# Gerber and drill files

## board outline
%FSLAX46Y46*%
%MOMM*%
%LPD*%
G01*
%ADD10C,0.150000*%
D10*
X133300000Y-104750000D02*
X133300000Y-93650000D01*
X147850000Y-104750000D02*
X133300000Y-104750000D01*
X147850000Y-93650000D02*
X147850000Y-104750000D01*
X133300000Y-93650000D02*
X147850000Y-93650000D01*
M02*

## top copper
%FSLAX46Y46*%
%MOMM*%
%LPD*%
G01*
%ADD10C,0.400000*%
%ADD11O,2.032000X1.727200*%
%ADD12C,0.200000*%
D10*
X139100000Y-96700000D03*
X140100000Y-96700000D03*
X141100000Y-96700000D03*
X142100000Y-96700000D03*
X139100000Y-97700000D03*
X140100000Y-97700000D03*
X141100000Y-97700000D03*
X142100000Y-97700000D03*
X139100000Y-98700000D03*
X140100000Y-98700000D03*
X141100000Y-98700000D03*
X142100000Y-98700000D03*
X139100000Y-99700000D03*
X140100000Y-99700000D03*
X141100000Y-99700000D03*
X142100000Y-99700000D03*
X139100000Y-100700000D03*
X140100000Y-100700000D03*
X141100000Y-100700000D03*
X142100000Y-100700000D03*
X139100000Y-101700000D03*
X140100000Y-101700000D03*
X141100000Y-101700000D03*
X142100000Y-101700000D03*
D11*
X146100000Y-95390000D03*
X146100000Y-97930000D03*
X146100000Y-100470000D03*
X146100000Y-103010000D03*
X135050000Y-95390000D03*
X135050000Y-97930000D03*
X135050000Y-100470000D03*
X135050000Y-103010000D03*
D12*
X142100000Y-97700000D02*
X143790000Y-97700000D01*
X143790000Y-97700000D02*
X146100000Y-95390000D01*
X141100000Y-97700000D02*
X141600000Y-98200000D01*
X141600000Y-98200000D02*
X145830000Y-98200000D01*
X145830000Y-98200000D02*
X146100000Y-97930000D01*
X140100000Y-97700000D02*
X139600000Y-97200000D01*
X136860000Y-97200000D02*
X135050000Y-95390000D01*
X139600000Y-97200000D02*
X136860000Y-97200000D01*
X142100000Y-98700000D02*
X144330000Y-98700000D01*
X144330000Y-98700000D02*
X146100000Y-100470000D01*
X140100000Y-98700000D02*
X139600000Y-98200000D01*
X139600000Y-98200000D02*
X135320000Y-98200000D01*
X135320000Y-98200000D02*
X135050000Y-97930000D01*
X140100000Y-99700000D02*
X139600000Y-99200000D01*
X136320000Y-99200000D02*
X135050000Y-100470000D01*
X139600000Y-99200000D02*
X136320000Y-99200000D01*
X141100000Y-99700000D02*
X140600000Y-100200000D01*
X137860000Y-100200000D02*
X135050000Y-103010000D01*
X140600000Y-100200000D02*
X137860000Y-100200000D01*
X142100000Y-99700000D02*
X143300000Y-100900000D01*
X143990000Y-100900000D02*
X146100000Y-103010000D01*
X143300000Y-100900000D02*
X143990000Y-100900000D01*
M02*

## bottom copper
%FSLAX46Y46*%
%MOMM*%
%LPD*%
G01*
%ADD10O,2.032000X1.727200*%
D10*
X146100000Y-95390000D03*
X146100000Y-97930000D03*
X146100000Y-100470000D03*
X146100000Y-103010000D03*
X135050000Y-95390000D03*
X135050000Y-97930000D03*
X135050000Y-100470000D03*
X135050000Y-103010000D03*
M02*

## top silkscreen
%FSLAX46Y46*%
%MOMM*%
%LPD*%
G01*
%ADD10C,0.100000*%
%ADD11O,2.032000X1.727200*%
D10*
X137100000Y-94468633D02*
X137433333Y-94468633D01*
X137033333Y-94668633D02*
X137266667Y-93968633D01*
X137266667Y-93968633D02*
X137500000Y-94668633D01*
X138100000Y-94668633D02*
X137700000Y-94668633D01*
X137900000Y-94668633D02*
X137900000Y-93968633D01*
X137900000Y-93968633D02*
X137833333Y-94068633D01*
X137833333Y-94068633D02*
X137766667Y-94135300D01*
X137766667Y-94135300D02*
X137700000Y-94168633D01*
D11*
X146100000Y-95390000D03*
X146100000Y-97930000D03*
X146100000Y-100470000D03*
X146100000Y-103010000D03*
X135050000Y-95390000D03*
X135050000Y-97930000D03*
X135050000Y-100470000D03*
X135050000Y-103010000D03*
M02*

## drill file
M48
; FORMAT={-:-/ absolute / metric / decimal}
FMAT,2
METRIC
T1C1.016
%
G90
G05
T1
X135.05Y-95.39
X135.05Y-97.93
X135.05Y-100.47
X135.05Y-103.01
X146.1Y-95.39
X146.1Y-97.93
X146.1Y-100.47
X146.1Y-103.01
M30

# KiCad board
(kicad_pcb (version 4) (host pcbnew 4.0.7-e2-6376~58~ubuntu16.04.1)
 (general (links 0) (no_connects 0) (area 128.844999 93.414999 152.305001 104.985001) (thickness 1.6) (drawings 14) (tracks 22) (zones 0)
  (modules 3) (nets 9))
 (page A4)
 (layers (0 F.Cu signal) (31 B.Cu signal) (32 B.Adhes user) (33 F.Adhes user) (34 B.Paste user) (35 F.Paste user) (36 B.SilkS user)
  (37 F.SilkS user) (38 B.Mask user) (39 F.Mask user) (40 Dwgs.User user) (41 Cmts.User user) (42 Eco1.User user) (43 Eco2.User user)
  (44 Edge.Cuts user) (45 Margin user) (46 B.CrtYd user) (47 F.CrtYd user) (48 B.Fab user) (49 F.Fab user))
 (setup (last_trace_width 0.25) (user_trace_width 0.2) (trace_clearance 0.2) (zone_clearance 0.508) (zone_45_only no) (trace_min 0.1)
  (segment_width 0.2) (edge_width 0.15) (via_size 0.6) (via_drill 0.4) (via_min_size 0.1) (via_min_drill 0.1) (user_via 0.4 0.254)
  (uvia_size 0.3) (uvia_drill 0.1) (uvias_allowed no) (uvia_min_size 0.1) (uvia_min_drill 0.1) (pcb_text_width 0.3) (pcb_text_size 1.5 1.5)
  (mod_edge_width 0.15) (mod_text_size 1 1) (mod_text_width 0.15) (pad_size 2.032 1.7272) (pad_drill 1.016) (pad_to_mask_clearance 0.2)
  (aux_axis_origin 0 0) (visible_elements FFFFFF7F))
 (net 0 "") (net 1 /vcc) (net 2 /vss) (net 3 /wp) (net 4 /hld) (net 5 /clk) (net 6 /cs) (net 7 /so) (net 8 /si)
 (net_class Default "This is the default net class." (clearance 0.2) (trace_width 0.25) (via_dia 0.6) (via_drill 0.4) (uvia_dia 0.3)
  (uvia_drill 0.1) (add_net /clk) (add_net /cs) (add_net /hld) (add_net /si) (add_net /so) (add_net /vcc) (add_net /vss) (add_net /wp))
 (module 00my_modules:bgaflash (layer F.Cu) (at 140.6 99.2)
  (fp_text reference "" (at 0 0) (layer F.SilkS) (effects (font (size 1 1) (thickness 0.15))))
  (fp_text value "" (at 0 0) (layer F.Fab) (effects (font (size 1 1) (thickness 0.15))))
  (pad A1 smd circle (at -1.5 -2.5) (size 0.4 0.4) (layers F.Cu F.Paste F.Mask))
  (pad A2 smd circle (at -0.5 -2.5) (size 0.4 0.4) (layers F.Cu F.Paste F.Mask))
  (pad A3 smd circle (at 0.5 -2.5) (size 0.4 0.4) (layers F.Cu F.Paste F.Mask))
  (pad A4 smd circle (at 1.5 -2.5) (size 0.4 0.4) (layers F.Cu F.Paste F.Mask))
  (pad B1 smd circle (at -1.5 -1.5) (size 0.4 0.4) (layers F.Cu F.Paste F.Mask))
  (pad CLK smd circle (at -0.5 -1.5) (size 0.4 0.4) (layers F.Cu F.Paste F.Mask))
  (pad VSS smd circle (at 0.5 -1.5) (size 0.4 0.4) (layers F.Cu F.Paste F.Mask))
  (pad VCC smd circle (at 1.5 -1.5) (size 0.4 0.4) (layers F.Cu F.Paste F.Mask))
  (pad C1 smd circle (at -1.5 -0.5) (size 0.4 0.4) (layers F.Cu F.Paste F.Mask))
  (pad CS smd circle (at -0.5 -0.5) (size 0.4 0.4) (layers F.Cu F.Paste F.Mask))
  (pad C3 smd circle (at 0.5 -0.5) (size 0.4 0.4) (layers F.Cu F.Paste F.Mask))
  (pad WP smd circle (at 1.5 -0.5) (size 0.4 0.4) (layers F.Cu F.Paste F.Mask))
  (pad D1 smd circle (at -1.5 0.5) (size 0.4 0.4) (layers F.Cu F.Paste F.Mask))
  (pad SO smd circle (at -0.5 0.5) (size 0.4 0.4) (layers F.Cu F.Paste F.Mask))
  (pad SI smd circle (at 0.5 0.5) (size 0.4 0.4) (layers F.Cu F.Paste F.Mask))
  (pad HLD smd circle (at 1.5 0.5) (size 0.4 0.4) (layers F.Cu F.Paste F.Mask))
  (pad E1 smd circle (at -1.5 1.5) (size 0.4 0.4) (layers F.Cu F.Paste F.Mask))
  (pad E2 smd circle (at -0.5 1.5) (size 0.4 0.4) (layers F.Cu F.Paste F.Mask))
  (pad E3 smd circle (at 0.5 1.5) (size 0.4 0.4) (layers F.Cu F.Paste F.Mask))
  (pad E4 smd circle (at 1.5 1.5) (size 0.4 0.4) (layers F.Cu F.Paste F.Mask))
  (pad F1 smd circle (at -1.5 2.5) (size 0.4 0.4) (layers F.Cu F.Paste F.Mask))
  (pad F2 smd circle (at -0.5 2.5) (size 0.4 0.4) (layers F.Cu F.Paste F.Mask))
  (pad F3 smd circle (at 0.5 2.5) (size 0.4 0.4) (layers F.Cu F.Paste F.Mask))
  (pad F4 smd circle (at 1.5 2.5) (size 0.4 0.4) (layers F.Cu F.Paste F.Mask)))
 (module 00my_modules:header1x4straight (layer F.Cu) (at 146.1 99.2)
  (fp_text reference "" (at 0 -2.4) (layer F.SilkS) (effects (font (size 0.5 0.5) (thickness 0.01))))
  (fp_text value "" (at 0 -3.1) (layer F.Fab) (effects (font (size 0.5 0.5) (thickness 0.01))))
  (pad 1 thru_hole oval (at 0 -3.81) (size 2.032 1.7272) (drill 1.016) (layers *.Cu *.Mask F.SilkS) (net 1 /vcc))
  (pad 2 thru_hole oval (at 0 -1.27) (size 2.032 1.7272) (drill 1.016) (layers *.Cu *.Mask F.SilkS) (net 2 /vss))
  (pad 3 thru_hole oval (at 0 1.27) (size 2.032 1.7272) (drill 1.016) (layers *.Cu *.Mask F.SilkS) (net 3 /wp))
  (pad 4 thru_hole oval (at 0 3.81) (size 2.032 1.7272) (drill 1.016) (layers *.Cu *.Mask F.SilkS) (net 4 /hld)))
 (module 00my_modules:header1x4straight (layer F.Cu) (at 135.05 99.2)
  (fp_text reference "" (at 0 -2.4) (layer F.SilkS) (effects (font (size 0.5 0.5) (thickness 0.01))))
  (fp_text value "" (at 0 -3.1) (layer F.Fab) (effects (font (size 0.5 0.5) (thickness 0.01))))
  (pad 1 thru_hole oval (at 0 -3.81) (size 2.032 1.7272) (drill 1.016) (layers *.Cu *.Mask F.SilkS) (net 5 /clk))
  (pad 2 thru_hole oval (at 0 -1.27) (size 2.032 1.7272) (drill 1.016) (layers *.Cu *.Mask F.SilkS) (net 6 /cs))
  (pad 3 thru_hole oval (at 0 1.27) (size 2.032 1.7272) (drill 1.016) (layers *.Cu *.Mask F.SilkS) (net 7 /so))
  (pad 4 thru_hole oval (at 0 3.81) (size 2.032 1.7272) (drill 1.016) (layers *.Cu *.Mask F.SilkS) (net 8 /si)))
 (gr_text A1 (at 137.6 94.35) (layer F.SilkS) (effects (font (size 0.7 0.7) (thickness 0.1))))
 (gr_line (start 133.3 104.75) (end 133.3 93.65) (angle 90) (layer Edge.Cuts) (width 0.15))
 (gr_line (start 147.85 104.75) (end 133.3 104.75) (angle 90) (layer Edge.Cuts) (width 0.15))
 (gr_line (start 147.85 93.65) (end 147.85 104.75) (angle 90) (layer Edge.Cuts) (width 0.15))
 (gr_line (start 133.3 93.65) (end 147.85 93.65) (angle 90) (layer Edge.Cuts) (width 0.15))
 (segment (start 142.1 97.7) (end 143.79 97.7) (width 0.2) (layer F.Cu) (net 1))
 (segment (start 143.79 97.7) (end 146.1 95.39) (width 0.2) (layer F.Cu) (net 1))
 (segment (start 141.1 97.7) (end 141.6 98.2) (width 0.2) (layer F.Cu) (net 2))
 (segment (start 141.6 98.2) (end 145.83 98.2) (width 0.2) (layer F.Cu) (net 2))
 (segment (start 145.83 98.2) (end 146.1 97.93) (width 0.2) (layer F.Cu) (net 2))
 (segment (start 140.1 97.7) (end 139.6 97.2) (width 0.2) (layer F.Cu) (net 5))
 (segment (start 136.86 97.2) (end 135.05 95.39) (width 0.2) (layer F.Cu) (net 5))
 (segment (start 139.6 97.2) (end 136.86 97.2) (width 0.2) (layer F.Cu) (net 5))
 (segment (start 142.1 98.7) (end 144.33 98.7) (width 0.2) (layer F.Cu) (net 3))
 (segment (start 144.33 98.7) (end 146.1 100.47) (width 0.2) (layer F.Cu) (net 3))
 (segment (start 140.1 98.7) (end 139.6 98.2) (width 0.2) (layer F.Cu) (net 6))
 (segment (start 139.6 98.2) (end 135.32 98.2) (width 0.2) (layer F.Cu) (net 6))
 (segment (start 135.32 98.2) (end 135.05 97.93) (width 0.2) (layer F.Cu) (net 6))
 (segment (start 140.1 99.7) (end 139.6 99.2) (width 0.2) (layer F.Cu) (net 7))
 (segment (start 136.32 99.2) (end 135.05 100.47) (width 0.2) (layer F.Cu) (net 7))
 (segment (start 139.6 99.2) (end 136.32 99.2) (width 0.2) (layer F.Cu) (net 7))
 (segment (start 141.1 99.7) (end 140.6 100.2) (width 0.2) (layer F.Cu) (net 8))
 (segment (start 137.86 100.2) (end 135.05 103.01) (width 0.2) (layer F.Cu) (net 8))
 (segment (start 140.6 100.2) (end 137.86 100.2) (width 0.2) (layer F.Cu) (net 8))
 (segment (start 142.1 99.7) (end 143.3 100.9) (width 0.2) (layer F.Cu) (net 4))
 (segment (start 143.99 100.9) (end 146.1 103.01) (width 0.2) (layer F.Cu) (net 4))
 (segment (start 143.3 100.9) (end 143.99 100.9) (width 0.2) (layer F.Cu) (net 4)))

